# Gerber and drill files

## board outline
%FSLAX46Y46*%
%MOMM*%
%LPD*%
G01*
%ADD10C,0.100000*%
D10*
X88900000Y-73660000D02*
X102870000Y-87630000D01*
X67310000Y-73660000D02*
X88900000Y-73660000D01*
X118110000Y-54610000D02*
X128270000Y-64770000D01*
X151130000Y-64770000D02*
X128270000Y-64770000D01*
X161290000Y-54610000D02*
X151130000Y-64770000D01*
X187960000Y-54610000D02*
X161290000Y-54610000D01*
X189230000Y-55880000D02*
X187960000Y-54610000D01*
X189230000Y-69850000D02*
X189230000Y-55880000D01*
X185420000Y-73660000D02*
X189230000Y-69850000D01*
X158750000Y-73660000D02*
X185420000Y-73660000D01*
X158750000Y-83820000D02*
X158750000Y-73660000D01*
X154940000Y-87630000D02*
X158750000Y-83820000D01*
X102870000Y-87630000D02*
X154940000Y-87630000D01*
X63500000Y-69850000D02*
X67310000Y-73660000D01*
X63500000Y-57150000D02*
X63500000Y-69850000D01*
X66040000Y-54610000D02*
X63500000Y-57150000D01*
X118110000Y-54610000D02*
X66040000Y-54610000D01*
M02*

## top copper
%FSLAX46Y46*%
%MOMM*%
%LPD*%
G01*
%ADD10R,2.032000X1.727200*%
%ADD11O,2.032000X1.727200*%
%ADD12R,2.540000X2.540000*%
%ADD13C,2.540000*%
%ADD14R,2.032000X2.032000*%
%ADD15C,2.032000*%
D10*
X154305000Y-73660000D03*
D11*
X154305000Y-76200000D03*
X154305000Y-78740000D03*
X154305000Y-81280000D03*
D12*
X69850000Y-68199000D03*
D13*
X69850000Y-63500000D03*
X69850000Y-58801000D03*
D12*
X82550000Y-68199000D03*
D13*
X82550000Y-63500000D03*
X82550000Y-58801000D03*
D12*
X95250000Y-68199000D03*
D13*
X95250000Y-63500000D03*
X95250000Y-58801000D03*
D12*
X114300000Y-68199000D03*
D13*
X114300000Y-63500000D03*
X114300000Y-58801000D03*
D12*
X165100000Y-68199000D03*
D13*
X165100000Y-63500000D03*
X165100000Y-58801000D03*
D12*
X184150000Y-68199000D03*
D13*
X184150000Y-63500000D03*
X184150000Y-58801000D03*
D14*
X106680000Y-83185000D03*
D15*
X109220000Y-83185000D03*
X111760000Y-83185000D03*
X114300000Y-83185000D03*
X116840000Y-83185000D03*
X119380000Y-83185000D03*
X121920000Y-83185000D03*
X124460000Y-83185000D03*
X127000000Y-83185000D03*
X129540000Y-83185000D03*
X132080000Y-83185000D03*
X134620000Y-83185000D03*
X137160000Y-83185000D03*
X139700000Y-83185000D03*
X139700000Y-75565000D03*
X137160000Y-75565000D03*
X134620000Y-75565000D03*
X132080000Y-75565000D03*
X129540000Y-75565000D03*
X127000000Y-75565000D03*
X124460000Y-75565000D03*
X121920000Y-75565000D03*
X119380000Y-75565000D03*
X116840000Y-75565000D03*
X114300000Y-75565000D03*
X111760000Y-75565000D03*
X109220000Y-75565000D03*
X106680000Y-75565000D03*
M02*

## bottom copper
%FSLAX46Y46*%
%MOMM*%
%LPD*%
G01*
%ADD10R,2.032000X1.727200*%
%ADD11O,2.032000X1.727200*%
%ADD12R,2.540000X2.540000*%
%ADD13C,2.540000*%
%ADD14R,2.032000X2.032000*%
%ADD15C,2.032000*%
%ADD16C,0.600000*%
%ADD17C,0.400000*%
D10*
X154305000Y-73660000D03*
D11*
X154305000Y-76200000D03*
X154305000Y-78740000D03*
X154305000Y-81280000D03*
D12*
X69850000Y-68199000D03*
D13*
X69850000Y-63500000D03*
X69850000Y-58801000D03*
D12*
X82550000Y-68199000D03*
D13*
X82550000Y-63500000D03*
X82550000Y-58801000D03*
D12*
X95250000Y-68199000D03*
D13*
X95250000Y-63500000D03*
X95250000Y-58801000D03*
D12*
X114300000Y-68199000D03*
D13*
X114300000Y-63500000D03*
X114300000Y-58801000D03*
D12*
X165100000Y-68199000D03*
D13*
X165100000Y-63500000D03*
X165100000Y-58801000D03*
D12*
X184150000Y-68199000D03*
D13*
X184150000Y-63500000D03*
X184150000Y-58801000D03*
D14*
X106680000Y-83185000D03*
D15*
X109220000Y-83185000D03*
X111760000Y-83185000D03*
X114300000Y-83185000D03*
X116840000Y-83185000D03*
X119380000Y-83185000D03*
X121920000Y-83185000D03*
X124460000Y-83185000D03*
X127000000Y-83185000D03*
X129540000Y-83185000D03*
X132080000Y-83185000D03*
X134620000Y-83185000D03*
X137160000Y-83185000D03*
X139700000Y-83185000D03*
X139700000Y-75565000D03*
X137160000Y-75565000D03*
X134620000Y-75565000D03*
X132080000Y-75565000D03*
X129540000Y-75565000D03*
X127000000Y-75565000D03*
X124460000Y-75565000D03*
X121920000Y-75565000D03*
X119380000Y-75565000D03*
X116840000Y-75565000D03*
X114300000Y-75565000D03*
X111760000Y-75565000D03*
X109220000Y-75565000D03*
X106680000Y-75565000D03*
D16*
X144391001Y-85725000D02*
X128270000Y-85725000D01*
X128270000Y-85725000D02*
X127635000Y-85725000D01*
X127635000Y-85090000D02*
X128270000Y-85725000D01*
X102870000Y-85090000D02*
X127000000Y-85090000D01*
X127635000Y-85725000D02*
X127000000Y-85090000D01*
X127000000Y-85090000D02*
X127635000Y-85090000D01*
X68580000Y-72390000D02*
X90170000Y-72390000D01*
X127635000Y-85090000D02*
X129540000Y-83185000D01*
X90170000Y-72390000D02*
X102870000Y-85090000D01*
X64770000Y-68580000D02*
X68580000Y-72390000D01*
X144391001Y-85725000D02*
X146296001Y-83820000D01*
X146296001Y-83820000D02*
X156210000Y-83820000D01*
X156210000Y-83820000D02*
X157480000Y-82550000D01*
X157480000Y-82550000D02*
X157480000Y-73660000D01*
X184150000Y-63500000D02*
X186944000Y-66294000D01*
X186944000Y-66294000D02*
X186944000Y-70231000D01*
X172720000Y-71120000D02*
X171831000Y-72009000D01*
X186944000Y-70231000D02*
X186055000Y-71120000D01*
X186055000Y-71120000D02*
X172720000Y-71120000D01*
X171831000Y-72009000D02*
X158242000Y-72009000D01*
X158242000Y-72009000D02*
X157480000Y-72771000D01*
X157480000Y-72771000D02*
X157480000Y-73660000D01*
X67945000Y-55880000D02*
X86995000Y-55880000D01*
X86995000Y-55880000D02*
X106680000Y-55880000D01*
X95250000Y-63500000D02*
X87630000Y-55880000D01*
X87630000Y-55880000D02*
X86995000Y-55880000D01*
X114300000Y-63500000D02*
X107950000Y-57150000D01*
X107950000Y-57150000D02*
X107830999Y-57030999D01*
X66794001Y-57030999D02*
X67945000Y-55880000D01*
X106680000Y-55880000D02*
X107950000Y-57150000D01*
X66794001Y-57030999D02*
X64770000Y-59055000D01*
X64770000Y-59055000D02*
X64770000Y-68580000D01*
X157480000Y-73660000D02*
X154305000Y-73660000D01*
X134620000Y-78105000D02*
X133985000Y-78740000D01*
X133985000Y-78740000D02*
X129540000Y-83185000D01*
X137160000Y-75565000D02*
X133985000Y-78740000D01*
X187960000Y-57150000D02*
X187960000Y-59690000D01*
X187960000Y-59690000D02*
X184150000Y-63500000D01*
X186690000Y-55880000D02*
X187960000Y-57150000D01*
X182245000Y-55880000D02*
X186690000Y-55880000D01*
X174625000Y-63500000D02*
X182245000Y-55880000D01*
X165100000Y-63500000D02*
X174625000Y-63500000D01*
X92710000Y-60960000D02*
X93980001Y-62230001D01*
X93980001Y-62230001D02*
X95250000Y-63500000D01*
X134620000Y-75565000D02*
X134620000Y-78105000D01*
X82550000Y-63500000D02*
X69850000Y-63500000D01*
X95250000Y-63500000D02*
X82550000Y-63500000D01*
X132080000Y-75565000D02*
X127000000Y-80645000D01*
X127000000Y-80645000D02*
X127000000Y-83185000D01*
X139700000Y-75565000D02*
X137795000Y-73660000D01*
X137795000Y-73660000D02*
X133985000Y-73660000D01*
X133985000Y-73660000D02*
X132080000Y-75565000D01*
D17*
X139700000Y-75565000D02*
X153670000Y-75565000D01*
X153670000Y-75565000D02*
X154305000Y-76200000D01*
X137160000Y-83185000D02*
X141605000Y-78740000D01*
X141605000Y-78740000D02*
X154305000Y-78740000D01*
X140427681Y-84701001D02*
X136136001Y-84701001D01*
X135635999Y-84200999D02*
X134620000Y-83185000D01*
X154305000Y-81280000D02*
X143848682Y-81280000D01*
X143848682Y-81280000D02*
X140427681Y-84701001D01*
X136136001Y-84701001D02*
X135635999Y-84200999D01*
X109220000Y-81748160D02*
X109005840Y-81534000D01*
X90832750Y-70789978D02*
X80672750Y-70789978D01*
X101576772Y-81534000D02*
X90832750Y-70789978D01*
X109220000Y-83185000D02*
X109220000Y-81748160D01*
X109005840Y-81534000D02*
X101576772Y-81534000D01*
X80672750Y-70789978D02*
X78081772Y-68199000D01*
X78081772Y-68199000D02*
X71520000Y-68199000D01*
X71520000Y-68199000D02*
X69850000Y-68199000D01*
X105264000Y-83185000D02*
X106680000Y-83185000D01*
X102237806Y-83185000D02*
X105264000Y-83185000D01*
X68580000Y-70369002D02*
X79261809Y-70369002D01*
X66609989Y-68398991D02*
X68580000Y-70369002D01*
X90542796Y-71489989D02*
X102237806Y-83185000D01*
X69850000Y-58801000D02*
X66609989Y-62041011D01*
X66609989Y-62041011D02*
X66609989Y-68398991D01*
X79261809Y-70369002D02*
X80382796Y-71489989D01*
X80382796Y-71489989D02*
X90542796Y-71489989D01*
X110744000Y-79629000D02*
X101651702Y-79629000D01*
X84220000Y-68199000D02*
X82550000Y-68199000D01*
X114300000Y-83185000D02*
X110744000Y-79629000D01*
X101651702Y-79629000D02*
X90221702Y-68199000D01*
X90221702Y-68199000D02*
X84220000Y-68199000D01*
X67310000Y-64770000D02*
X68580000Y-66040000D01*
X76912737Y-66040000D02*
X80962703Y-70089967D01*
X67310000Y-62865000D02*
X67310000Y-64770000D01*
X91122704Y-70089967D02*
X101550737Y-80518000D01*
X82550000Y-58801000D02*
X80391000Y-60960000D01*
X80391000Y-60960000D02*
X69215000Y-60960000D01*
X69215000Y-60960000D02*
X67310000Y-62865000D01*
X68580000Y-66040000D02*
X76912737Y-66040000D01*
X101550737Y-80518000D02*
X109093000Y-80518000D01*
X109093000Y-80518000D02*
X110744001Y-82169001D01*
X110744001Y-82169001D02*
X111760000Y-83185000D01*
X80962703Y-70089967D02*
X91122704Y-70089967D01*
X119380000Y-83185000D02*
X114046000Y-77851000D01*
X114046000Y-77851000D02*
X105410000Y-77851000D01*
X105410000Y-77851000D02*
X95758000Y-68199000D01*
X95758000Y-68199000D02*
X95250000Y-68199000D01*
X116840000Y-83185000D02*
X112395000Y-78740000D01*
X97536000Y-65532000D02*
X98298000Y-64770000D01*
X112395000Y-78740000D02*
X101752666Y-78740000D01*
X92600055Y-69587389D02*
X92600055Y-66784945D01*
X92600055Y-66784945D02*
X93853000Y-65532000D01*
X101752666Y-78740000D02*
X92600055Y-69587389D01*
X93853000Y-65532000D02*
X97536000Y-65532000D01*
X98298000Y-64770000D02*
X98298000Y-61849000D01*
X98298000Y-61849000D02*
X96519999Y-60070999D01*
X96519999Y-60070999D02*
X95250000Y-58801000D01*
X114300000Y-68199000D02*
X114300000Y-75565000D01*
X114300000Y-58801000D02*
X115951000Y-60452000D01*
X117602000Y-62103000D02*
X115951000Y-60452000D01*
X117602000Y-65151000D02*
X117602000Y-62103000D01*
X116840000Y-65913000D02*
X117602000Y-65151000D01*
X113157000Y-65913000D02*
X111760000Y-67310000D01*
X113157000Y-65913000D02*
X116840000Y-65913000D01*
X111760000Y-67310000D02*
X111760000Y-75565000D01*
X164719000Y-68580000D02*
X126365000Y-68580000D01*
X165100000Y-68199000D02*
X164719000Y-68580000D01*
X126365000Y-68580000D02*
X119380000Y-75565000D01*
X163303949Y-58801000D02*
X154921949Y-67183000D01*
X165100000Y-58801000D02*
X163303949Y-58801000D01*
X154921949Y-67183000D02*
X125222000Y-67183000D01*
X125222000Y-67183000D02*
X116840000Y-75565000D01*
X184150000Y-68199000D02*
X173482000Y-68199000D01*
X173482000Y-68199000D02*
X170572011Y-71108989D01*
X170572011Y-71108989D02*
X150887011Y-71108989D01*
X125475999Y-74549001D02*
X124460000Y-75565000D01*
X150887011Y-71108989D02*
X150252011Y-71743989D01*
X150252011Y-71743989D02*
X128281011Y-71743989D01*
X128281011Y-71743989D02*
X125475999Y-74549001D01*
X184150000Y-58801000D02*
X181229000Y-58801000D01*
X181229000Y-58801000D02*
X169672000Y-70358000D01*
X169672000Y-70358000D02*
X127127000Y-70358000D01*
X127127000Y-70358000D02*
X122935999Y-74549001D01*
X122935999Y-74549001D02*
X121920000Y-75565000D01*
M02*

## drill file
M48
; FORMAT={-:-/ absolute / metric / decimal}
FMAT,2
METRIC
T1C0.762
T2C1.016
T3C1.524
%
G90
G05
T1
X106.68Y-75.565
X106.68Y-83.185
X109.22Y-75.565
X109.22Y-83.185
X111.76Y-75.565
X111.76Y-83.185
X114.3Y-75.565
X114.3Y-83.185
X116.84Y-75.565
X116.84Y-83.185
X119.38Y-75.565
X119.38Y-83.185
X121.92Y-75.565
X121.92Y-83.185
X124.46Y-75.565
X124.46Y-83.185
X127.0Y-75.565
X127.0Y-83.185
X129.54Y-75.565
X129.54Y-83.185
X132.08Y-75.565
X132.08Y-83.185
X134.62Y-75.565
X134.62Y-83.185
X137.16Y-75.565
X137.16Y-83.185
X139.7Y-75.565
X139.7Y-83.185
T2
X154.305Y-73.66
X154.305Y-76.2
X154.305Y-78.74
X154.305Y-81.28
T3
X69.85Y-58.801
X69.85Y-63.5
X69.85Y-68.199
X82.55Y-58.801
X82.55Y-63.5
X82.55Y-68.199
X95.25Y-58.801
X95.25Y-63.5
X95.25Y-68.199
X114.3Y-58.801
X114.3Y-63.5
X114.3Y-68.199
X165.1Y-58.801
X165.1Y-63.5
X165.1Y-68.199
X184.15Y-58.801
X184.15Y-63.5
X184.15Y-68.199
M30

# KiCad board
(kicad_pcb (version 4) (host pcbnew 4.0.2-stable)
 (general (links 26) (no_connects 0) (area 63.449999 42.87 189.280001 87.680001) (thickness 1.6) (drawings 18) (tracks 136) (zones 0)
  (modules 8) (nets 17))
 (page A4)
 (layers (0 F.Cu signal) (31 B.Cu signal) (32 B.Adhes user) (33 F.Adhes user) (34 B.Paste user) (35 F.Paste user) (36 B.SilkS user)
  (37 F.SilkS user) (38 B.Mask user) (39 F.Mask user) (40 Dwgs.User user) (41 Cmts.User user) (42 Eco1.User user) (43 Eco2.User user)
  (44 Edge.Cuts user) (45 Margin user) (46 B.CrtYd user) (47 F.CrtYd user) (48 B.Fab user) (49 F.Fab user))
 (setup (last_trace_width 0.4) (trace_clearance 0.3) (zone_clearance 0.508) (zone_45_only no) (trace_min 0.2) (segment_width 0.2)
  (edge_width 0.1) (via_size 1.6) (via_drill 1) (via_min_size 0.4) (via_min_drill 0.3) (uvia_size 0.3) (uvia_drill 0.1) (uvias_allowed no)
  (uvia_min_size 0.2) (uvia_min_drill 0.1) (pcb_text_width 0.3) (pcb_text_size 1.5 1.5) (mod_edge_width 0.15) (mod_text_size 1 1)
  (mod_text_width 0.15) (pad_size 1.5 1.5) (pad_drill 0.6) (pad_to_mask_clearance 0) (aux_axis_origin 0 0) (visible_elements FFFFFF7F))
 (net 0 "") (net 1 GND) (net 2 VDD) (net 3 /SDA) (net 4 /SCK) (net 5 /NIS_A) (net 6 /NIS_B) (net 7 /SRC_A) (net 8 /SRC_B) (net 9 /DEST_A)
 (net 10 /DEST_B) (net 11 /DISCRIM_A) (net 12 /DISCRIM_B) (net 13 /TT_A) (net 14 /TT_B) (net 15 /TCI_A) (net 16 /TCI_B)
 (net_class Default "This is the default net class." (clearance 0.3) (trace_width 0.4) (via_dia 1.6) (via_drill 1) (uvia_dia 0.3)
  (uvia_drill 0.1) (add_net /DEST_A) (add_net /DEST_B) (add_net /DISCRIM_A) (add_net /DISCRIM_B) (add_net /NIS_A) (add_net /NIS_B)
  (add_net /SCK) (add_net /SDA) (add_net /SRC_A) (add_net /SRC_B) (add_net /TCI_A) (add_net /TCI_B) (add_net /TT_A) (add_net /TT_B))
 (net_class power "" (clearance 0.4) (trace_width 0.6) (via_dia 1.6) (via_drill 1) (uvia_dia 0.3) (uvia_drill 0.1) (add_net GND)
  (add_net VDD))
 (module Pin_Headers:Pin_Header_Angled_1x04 (layer F.Cu) (at 154.305 73.66)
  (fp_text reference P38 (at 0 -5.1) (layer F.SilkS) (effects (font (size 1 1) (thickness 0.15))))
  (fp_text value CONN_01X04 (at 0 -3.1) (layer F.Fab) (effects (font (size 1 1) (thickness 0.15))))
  (pad 1 thru_hole rect (at 0 0) (size 2.032 1.7272) (drill 1.016) (layers *.Cu *.Mask F.SilkS) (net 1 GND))
  (pad 2 thru_hole oval (at 0 2.54) (size 2.032 1.7272) (drill 1.016) (layers *.Cu *.Mask F.SilkS) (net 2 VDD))
  (pad 3 thru_hole oval (at 0 5.08) (size 2.032 1.7272) (drill 1.016) (layers *.Cu *.Mask F.SilkS) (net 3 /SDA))
  (pad 4 thru_hole oval (at 0 7.62) (size 2.032 1.7272) (drill 1.016) (layers *.Cu *.Mask F.SilkS) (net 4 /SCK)))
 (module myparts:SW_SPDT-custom (layer F.Cu) (at 69.85 63.5 90)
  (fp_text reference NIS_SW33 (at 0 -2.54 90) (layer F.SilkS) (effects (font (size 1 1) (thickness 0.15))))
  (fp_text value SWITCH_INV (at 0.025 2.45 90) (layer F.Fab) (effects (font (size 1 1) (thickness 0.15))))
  (pad 1 thru_hole rect (at -4.699 0 90) (size 2.54 2.54) (drill 1.524) (layers *.Cu *.Mask F.SilkS) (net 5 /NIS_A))
  (pad 2 thru_hole circle (at 0 0 90) (size 2.54 2.54) (drill 1.524) (layers *.Cu *.Mask F.SilkS) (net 1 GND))
  (pad 3 thru_hole circle (at 4.699 0 90) (size 2.54 2.54) (drill 1.524) (layers *.Cu *.Mask F.SilkS) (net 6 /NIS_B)))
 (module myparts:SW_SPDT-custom (layer F.Cu) (at 82.55 63.5 90)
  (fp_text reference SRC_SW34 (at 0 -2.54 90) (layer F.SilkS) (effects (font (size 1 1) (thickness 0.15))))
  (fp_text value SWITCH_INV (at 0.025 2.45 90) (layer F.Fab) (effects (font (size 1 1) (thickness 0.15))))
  (pad 1 thru_hole rect (at -4.699 0 90) (size 2.54 2.54) (drill 1.524) (layers *.Cu *.Mask F.SilkS) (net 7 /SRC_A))
  (pad 2 thru_hole circle (at 0 0 90) (size 2.54 2.54) (drill 1.524) (layers *.Cu *.Mask F.SilkS) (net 1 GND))
  (pad 3 thru_hole circle (at 4.699 0 90) (size 2.54 2.54) (drill 1.524) (layers *.Cu *.Mask F.SilkS) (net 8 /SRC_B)))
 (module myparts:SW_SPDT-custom (layer F.Cu) (at 95.25 63.5 90)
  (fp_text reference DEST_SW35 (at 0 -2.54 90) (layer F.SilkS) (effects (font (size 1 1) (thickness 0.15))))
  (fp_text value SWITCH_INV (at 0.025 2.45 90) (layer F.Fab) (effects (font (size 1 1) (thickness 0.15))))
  (pad 1 thru_hole rect (at -4.699 0 90) (size 2.54 2.54) (drill 1.524) (layers *.Cu *.Mask F.SilkS) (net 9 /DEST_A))
  (pad 2 thru_hole circle (at 0 0 90) (size 2.54 2.54) (drill 1.524) (layers *.Cu *.Mask F.SilkS) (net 1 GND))
  (pad 3 thru_hole circle (at 4.699 0 90) (size 2.54 2.54) (drill 1.524) (layers *.Cu *.Mask F.SilkS) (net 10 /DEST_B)))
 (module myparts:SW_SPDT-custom (layer F.Cu) (at 114.3 63.5 90)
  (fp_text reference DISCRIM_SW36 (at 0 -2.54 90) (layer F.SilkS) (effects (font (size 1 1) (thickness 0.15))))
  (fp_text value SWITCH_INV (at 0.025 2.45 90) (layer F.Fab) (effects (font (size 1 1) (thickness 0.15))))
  (pad 1 thru_hole rect (at -4.699 0 90) (size 2.54 2.54) (drill 1.524) (layers *.Cu *.Mask F.SilkS) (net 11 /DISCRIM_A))
  (pad 2 thru_hole circle (at 0 0 90) (size 2.54 2.54) (drill 1.524) (layers *.Cu *.Mask F.SilkS) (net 1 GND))
  (pad 3 thru_hole circle (at 4.699 0 90) (size 2.54 2.54) (drill 1.524) (layers *.Cu *.Mask F.SilkS) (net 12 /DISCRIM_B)))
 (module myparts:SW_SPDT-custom (layer F.Cu) (at 165.1 63.5 90)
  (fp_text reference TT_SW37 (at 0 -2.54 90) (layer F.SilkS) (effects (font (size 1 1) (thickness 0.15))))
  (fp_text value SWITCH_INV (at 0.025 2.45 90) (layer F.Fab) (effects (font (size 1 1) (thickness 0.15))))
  (pad 1 thru_hole rect (at -4.699 0 90) (size 2.54 2.54) (drill 1.524) (layers *.Cu *.Mask F.SilkS) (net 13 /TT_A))
  (pad 2 thru_hole circle (at 0 0 90) (size 2.54 2.54) (drill 1.524) (layers *.Cu *.Mask F.SilkS) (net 1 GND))
  (pad 3 thru_hole circle (at 4.699 0 90) (size 2.54 2.54) (drill 1.524) (layers *.Cu *.Mask F.SilkS) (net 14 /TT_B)))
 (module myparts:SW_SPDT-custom (layer F.Cu) (at 184.15 63.5 90)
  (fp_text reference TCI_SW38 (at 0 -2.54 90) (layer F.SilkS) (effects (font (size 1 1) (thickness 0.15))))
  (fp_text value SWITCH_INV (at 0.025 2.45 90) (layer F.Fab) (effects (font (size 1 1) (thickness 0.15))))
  (pad 1 thru_hole rect (at -4.699 0 90) (size 2.54 2.54) (drill 1.524) (layers *.Cu *.Mask F.SilkS) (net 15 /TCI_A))
  (pad 2 thru_hole circle (at 0 0 90) (size 2.54 2.54) (drill 1.524) (layers *.Cu *.Mask F.SilkS) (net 1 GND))
  (pad 3 thru_hole circle (at 4.699 0 90) (size 2.54 2.54) (drill 1.524) (layers *.Cu *.Mask F.SilkS) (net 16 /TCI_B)))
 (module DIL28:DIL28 (layer F.Cu) (at 106.68 83.185)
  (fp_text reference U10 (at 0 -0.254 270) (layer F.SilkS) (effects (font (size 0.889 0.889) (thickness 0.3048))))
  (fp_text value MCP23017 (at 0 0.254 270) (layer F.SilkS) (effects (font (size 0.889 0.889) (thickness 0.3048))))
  (pad 1 thru_hole rect (at 0 0) (size 2.032 2.032) (drill 0.762) (layers *.Cu *.Mask F.SilkS) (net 6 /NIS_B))
  (pad 2 thru_hole circle (at 2.54 0) (size 2.032 2.032) (drill 0.762) (layers *.Cu *.Mask F.SilkS) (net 5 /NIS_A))
  (pad 3 thru_hole circle (at 5.08 0) (size 2.032 2.032) (drill 0.762) (layers *.Cu *.Mask F.SilkS) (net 8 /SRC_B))
  (pad 4 thru_hole circle (at 7.62 0) (size 2.032 2.032) (drill 0.762) (layers *.Cu *.Mask F.SilkS) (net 7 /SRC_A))
  (pad 5 thru_hole circle (at 10.16 0) (size 2.032 2.032) (drill 0.762) (layers *.Cu *.Mask F.SilkS) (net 10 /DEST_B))
  (pad 6 thru_hole circle (at 12.7 0) (size 2.032 2.032) (drill 0.762) (layers *.Cu *.Mask F.SilkS) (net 9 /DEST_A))
  (pad 7 thru_hole circle (at 15.24 0) (size 2.032 2.032) (drill 0.762) (layers *.Cu *.Mask F.SilkS))
  (pad 8 thru_hole circle (at 17.78 0) (size 2.032 2.032) (drill 0.762) (layers *.Cu *.Mask F.SilkS))
  (pad 9 thru_hole circle (at 20.32 0) (size 2.032 2.032) (drill 0.762) (layers *.Cu *.Mask F.SilkS) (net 2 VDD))
  (pad 10 thru_hole circle (at 22.86 0) (size 2.032 2.032) (drill 0.762) (layers *.Cu *.Mask F.SilkS) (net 1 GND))
  (pad 11 thru_hole circle (at 25.4 0) (size 2.032 2.032) (drill 0.762) (layers *.Cu *.Mask F.SilkS))
  (pad 12 thru_hole circle (at 27.94 0) (size 2.032 2.032) (drill 0.762) (layers *.Cu *.Mask F.SilkS) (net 4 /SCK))
  (pad 13 thru_hole circle (at 30.48 0) (size 2.032 2.032) (drill 0.762) (layers *.Cu *.Mask F.SilkS) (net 3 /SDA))
  (pad 14 thru_hole circle (at 33.02 0) (size 2.032 2.032) (drill 0.762) (layers *.Cu *.Mask F.SilkS))
  (pad 15 thru_hole circle (at 33.02 -7.62 180) (size 2.032 2.032) (drill 0.762) (layers *.Cu *.Mask F.SilkS) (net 2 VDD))
  (pad 16 thru_hole circle (at 30.48 -7.62 180) (size 2.032 2.032) (drill 0.762) (layers *.Cu *.Mask F.SilkS) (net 1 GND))
  (pad 17 thru_hole circle (at 27.94 -7.62 180) (size 2.032 2.032) (drill 0.762) (layers *.Cu *.Mask F.SilkS) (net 1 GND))
  (pad 18 thru_hole circle (at 25.4 -7.62 180) (size 2.032 2.032) (drill 0.762) (layers *.Cu *.Mask F.SilkS) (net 2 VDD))
  (pad 19 thru_hole circle (at 22.86 -7.62 180) (size 2.032 2.032) (drill 0.762) (layers *.Cu *.Mask F.SilkS))
  (pad 20 thru_hole circle (at 20.32 -7.62 180) (size 2.032 2.032) (drill 0.762) (layers *.Cu *.Mask F.SilkS))
  (pad 21 thru_hole circle (at 17.78 -7.62 180) (size 2.032 2.032) (drill 0.762) (layers *.Cu *.Mask F.SilkS) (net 15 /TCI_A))
  (pad 22 thru_hole circle (at 15.24 -7.62 180) (size 2.032 2.032) (drill 0.762) (layers *.Cu *.Mask F.SilkS) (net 16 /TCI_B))
  (pad 23 thru_hole circle (at 12.7 -7.62 180) (size 2.032 2.032) (drill 0.762) (layers *.Cu *.Mask F.SilkS) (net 13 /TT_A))
  (pad 24 thru_hole circle (at 10.16 -7.62 180) (size 2.032 2.032) (drill 0.762) (layers *.Cu *.Mask F.SilkS) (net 14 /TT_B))
  (pad 25 thru_hole circle (at 7.62 -7.62 180) (size 2.032 2.032) (drill 0.762) (layers *.Cu *.Mask F.SilkS) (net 11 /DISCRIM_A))
  (pad 26 thru_hole circle (at 5.08 -7.62 180) (size 2.032 2.032) (drill 0.762) (layers *.Cu *.Mask F.SilkS) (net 12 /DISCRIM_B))
  (pad 27 thru_hole circle (at 2.54 -7.62 180) (size 2.032 2.032) (drill 0.762) (layers *.Cu *.Mask F.SilkS))
  (pad 28 thru_hole circle (at 0 -7.62 180) (size 2.032 2.032) (drill 0.762) (layers *.Cu *.Mask F.SilkS)))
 (gr_line (start 88.9 73.66) (end 102.87 87.63) (layer Edge.Cuts) (width 0.1))
 (gr_line (start 67.31 73.66) (end 88.9 73.66) (layer Edge.Cuts) (width 0.1))
 (gr_line (start 118.11 54.61) (end 128.27 64.77) (layer Edge.Cuts) (width 0.1))
 (gr_line (start 151.13 64.77) (end 128.27 64.77) (layer Edge.Cuts) (width 0.1))
 (gr_line (start 161.29 54.61) (end 151.13 64.77) (layer Edge.Cuts) (width 0.1))
 (gr_line (start 187.96 54.61) (end 161.29 54.61) (layer Edge.Cuts) (width 0.1))
 (gr_line (start 189.23 55.88) (end 187.96 54.61) (layer Edge.Cuts) (width 0.1))
 (gr_line (start 189.23 69.85) (end 189.23 55.88) (layer Edge.Cuts) (width 0.1))
 (gr_line (start 185.42 73.66) (end 189.23 69.85) (layer Edge.Cuts) (width 0.1))
 (gr_line (start 158.75 73.66) (end 185.42 73.66) (layer Edge.Cuts) (width 0.1))
 (gr_line (start 158.75 83.82) (end 158.75 73.66) (layer Edge.Cuts) (width 0.1))
 (gr_line (start 154.94 87.63) (end 158.75 83.82) (layer Edge.Cuts) (width 0.1))
 (gr_line (start 102.87 87.63) (end 154.94 87.63) (layer Edge.Cuts) (width 0.1))
 (gr_line (start 63.5 69.85) (end 67.31 73.66) (layer Edge.Cuts) (width 0.1))
 (gr_line (start 63.5 57.15) (end 63.5 69.85) (layer Edge.Cuts) (width 0.1))
 (gr_line (start 66.04 54.61) (end 63.5 57.15) (layer Edge.Cuts) (width 0.1))
 (gr_line (start 118.11 54.61) (end 66.04 54.61) (layer Edge.Cuts) (width 0.1))
 (segment (start 144.391001 85.725) (end 128.27 85.725) (width 0.6) (layer B.Cu) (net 1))
 (segment (start 128.27 85.725) (end 127.635 85.725) (width 0.6) (layer B.Cu) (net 1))
 (segment (start 127.635 85.09) (end 128.27 85.725) (width 0.6) (layer B.Cu) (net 1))
 (segment (start 102.87 85.09) (end 127 85.09) (width 0.6) (layer B.Cu) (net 1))
 (segment (start 127.635 85.725) (end 127 85.09) (width 0.6) (layer B.Cu) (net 1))
 (segment (start 127 85.09) (end 127.635 85.09) (width 0.6) (layer B.Cu) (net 1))
 (segment (start 68.58 72.39) (end 90.17 72.39) (width 0.6) (layer B.Cu) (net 1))
 (segment (start 127.635 85.09) (end 129.54 83.185) (width 0.6) (layer B.Cu) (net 1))
 (segment (start 90.17 72.39) (end 102.87 85.09) (width 0.6) (layer B.Cu) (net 1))
 (segment (start 64.77 68.58) (end 68.58 72.39) (width 0.6) (layer B.Cu) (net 1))
 (segment (start 144.391001 85.725) (end 146.296001 83.82) (width 0.6) (layer B.Cu) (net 1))
 (segment (start 146.296001 83.82) (end 156.21 83.82) (width 0.6) (layer B.Cu) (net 1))
 (segment (start 156.21 83.82) (end 157.48 82.55) (width 0.6) (layer B.Cu) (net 1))
 (segment (start 157.48 82.55) (end 157.48 73.66) (width 0.6) (layer B.Cu) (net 1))
 (segment (start 184.15 63.5) (end 186.944 66.294) (width 0.6) (layer B.Cu) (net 1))
 (segment (start 186.944 66.294) (end 186.944 70.231) (width 0.6) (layer B.Cu) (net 1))
 (segment (start 172.72 71.12) (end 171.831 72.009) (width 0.6) (layer B.Cu) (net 1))
 (segment (start 186.944 70.231) (end 186.055 71.12) (width 0.6) (layer B.Cu) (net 1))
 (segment (start 186.055 71.12) (end 172.72 71.12) (width 0.6) (layer B.Cu) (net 1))
 (segment (start 171.831 72.009) (end 158.242 72.009) (width 0.6) (layer B.Cu) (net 1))
 (segment (start 158.242 72.009) (end 157.48 72.771) (width 0.6) (layer B.Cu) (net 1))
 (segment (start 157.48 72.771) (end 157.48 73.66) (width 0.6) (layer B.Cu) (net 1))
 (segment (start 67.945 55.88) (end 86.995 55.88) (width 0.6) (layer B.Cu) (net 1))
 (segment (start 86.995 55.88) (end 106.68 55.88) (width 0.6) (layer B.Cu) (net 1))
 (segment (start 95.25 63.5) (end 87.63 55.88) (width 0.6) (layer B.Cu) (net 1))
 (segment (start 87.63 55.88) (end 86.995 55.88) (width 0.6) (layer B.Cu) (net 1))
 (segment (start 114.3 63.5) (end 107.95 57.15) (width 0.6) (layer B.Cu) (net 1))
 (segment (start 107.95 57.15) (end 107.830999 57.030999) (width 0.6) (layer B.Cu) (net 1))
 (segment (start 66.794001 57.030999) (end 67.945 55.88) (width 0.6) (layer B.Cu) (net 1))
 (segment (start 106.68 55.88) (end 107.95 57.15) (width 0.6) (layer B.Cu) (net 1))
 (segment (start 66.794001 57.030999) (end 64.77 59.055) (width 0.6) (layer B.Cu) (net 1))
 (segment (start 64.77 59.055) (end 64.77 68.58) (width 0.6) (layer B.Cu) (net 1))
 (segment (start 157.48 73.66) (end 154.305 73.66) (width 0.6) (layer B.Cu) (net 1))
 (segment (start 134.62 78.105) (end 133.985 78.74) (width 0.6) (layer B.Cu) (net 1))
 (segment (start 133.985 78.74) (end 129.54 83.185) (width 0.6) (layer B.Cu) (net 1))
 (segment (start 137.16 75.565) (end 133.985 78.74) (width 0.6) (layer B.Cu) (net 1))
 (segment (start 187.96 57.15) (end 187.96 59.69) (width 0.6) (layer B.Cu) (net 1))
 (segment (start 187.96 59.69) (end 184.15 63.5) (width 0.6) (layer B.Cu) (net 1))
 (segment (start 186.69 55.88) (end 187.96 57.15) (width 0.6) (layer B.Cu) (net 1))
 (segment (start 182.245 55.88) (end 186.69 55.88) (width 0.6) (layer B.Cu) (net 1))
 (segment (start 174.625 63.5) (end 182.245 55.88) (width 0.6) (layer B.Cu) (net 1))
 (segment (start 165.1 63.5) (end 174.625 63.5) (width 0.6) (layer B.Cu) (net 1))
 (segment (start 92.71 60.96) (end 93.980001 62.230001) (width 0.6) (layer B.Cu) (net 1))
 (segment (start 93.980001 62.230001) (end 95.25 63.5) (width 0.6) (layer B.Cu) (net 1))
 (segment (start 134.62 75.565) (end 134.62 78.105) (width 0.6) (layer B.Cu) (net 1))
 (segment (start 82.55 63.5) (end 69.85 63.5) (width 0.6) (layer B.Cu) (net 1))
 (segment (start 95.25 63.5) (end 82.55 63.5) (width 0.6) (layer B.Cu) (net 1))
 (segment (start 132.08 75.565) (end 127 80.645) (width 0.6) (layer B.Cu) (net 2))
 (segment (start 127 80.645) (end 127 83.185) (width 0.6) (layer B.Cu) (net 2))
 (segment (start 139.7 75.565) (end 137.795 73.66) (width 0.6) (layer B.Cu) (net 2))
 (segment (start 137.795 73.66) (end 133.985 73.66) (width 0.6) (layer B.Cu) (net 2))
 (segment (start 133.985 73.66) (end 132.08 75.565) (width 0.6) (layer B.Cu) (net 2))
 (segment (start 139.7 75.565) (end 153.67 75.565) (width 0.4) (layer B.Cu) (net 2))
 (segment (start 153.67 75.565) (end 154.305 76.2) (width 0.4) (layer B.Cu) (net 2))
 (segment (start 137.16 83.185) (end 141.605 78.74) (width 0.4) (layer B.Cu) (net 3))
 (segment (start 141.605 78.74) (end 154.305 78.74) (width 0.4) (layer B.Cu) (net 3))
 (segment (start 140.427681 84.701001) (end 136.136001 84.701001) (width 0.4) (layer B.Cu) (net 4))
 (segment (start 135.635999 84.200999) (end 134.62 83.185) (width 0.4) (layer B.Cu) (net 4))
 (segment (start 154.305 81.28) (end 143.848682 81.28) (width 0.4) (layer B.Cu) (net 4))
 (segment (start 143.848682 81.28) (end 140.427681 84.701001) (width 0.4) (layer B.Cu) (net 4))
 (segment (start 136.136001 84.701001) (end 135.635999 84.200999) (width 0.4) (layer B.Cu) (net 4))
 (segment (start 109.22 81.74816) (end 109.00584 81.534) (width 0.4) (layer B.Cu) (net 5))
 (segment (start 90.83275 70.789978) (end 80.67275 70.789978) (width 0.4) (layer B.Cu) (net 5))
 (segment (start 101.576772 81.534) (end 90.83275 70.789978) (width 0.4) (layer B.Cu) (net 5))
 (segment (start 109.22 83.185) (end 109.22 81.74816) (width 0.4) (layer B.Cu) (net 5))
 (segment (start 109.00584 81.534) (end 101.576772 81.534) (width 0.4) (layer B.Cu) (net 5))
 (segment (start 80.67275 70.789978) (end 78.081772 68.199) (width 0.4) (layer B.Cu) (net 5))
 (segment (start 78.081772 68.199) (end 71.52 68.199) (width 0.4) (layer B.Cu) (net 5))
 (segment (start 71.52 68.199) (end 69.85 68.199) (width 0.4) (layer B.Cu) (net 5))
 (segment (start 105.264 83.185) (end 106.68 83.185) (width 0.4) (layer B.Cu) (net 6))
 (segment (start 102.237806 83.185) (end 105.264 83.185) (width 0.4) (layer B.Cu) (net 6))
 (segment (start 68.58 70.369002) (end 79.261809 70.369002) (width 0.4) (layer B.Cu) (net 6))
 (segment (start 66.609989 68.398991) (end 68.58 70.369002) (width 0.4) (layer B.Cu) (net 6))
 (segment (start 90.542796 71.489989) (end 102.237806 83.185) (width 0.4) (layer B.Cu) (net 6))
 (segment (start 69.85 58.801) (end 66.609989 62.041011) (width 0.4) (layer B.Cu) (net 6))
 (segment (start 66.609989 62.041011) (end 66.609989 68.398991) (width 0.4) (layer B.Cu) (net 6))
 (segment (start 79.261809 70.369002) (end 80.382796 71.489989) (width 0.4) (layer B.Cu) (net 6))
 (segment (start 80.382796 71.489989) (end 90.542796 71.489989) (width 0.4) (layer B.Cu) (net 6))
 (segment (start 110.744 79.629) (end 101.651702 79.629) (width 0.4) (layer B.Cu) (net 7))
 (segment (start 84.22 68.199) (end 82.55 68.199) (width 0.4) (layer B.Cu) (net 7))
 (segment (start 114.3 83.185) (end 110.744 79.629) (width 0.4) (layer B.Cu) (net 7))
 (segment (start 101.651702 79.629) (end 90.221702 68.199) (width 0.4) (layer B.Cu) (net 7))
 (segment (start 90.221702 68.199) (end 84.22 68.199) (width 0.4) (layer B.Cu) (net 7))
 (segment (start 67.31 64.77) (end 68.58 66.04) (width 0.4) (layer B.Cu) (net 8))
 (segment (start 76.912737 66.04) (end 80.962703 70.089967) (width 0.4) (layer B.Cu) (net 8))
 (segment (start 67.31 62.865) (end 67.31 64.77) (width 0.4) (layer B.Cu) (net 8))
 (segment (start 91.122704 70.089967) (end 101.550737 80.518) (width 0.4) (layer B.Cu) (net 8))
 (segment (start 82.55 58.801) (end 80.391 60.96) (width 0.4) (layer B.Cu) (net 8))
 (segment (start 80.391 60.96) (end 69.215 60.96) (width 0.4) (layer B.Cu) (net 8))
 (segment (start 69.215 60.96) (end 67.31 62.865) (width 0.4) (layer B.Cu) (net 8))
 (segment (start 68.58 66.04) (end 76.912737 66.04) (width 0.4) (layer B.Cu) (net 8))
 (segment (start 101.550737 80.518) (end 109.093 80.518) (width 0.4) (layer B.Cu) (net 8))
 (segment (start 109.093 80.518) (end 110.744001 82.169001) (width 0.4) (layer B.Cu) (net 8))
 (segment (start 110.744001 82.169001) (end 111.76 83.185) (width 0.4) (layer B.Cu) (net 8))
 (segment (start 80.962703 70.089967) (end 91.122704 70.089967) (width 0.4) (layer B.Cu) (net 8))
 (segment (start 119.38 83.185) (end 114.046 77.851) (width 0.4) (layer B.Cu) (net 9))
 (segment (start 114.046 77.851) (end 105.41 77.851) (width 0.4) (layer B.Cu) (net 9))
 (segment (start 105.41 77.851) (end 95.758 68.199) (width 0.4) (layer B.Cu) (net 9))
 (segment (start 95.758 68.199) (end 95.25 68.199) (width 0.4) (layer B.Cu) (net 9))
 (segment (start 116.84 83.185) (end 112.395 78.74) (width 0.4) (layer B.Cu) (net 10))
 (segment (start 97.536 65.532) (end 98.298 64.77) (width 0.4) (layer B.Cu) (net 10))
 (segment (start 112.395 78.74) (end 101.752666 78.74) (width 0.4) (layer B.Cu) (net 10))
 (segment (start 92.600055 69.587389) (end 92.600055 66.784945) (width 0.4) (layer B.Cu) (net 10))
 (segment (start 92.600055 66.784945) (end 93.853 65.532) (width 0.4) (layer B.Cu) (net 10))
 (segment (start 101.752666 78.74) (end 92.600055 69.587389) (width 0.4) (layer B.Cu) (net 10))
 (segment (start 93.853 65.532) (end 97.536 65.532) (width 0.4) (layer B.Cu) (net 10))
 (segment (start 98.298 64.77) (end 98.298 61.849) (width 0.4) (layer B.Cu) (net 10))
 (segment (start 98.298 61.849) (end 96.519999 60.070999) (width 0.4) (layer B.Cu) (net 10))
 (segment (start 96.519999 60.070999) (end 95.25 58.801) (width 0.4) (layer B.Cu) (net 10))
 (segment (start 114.3 68.199) (end 114.3 75.565) (width 0.4) (layer B.Cu) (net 11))
 (segment (start 114.3 58.801) (end 115.951 60.452) (width 0.4) (layer B.Cu) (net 12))
 (segment (start 117.602 62.103) (end 115.951 60.452) (width 0.4) (layer B.Cu) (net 12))
 (segment (start 117.602 65.151) (end 117.602 62.103) (width 0.4) (layer B.Cu) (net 12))
 (segment (start 116.84 65.913) (end 117.602 65.151) (width 0.4) (layer B.Cu) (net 12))
 (segment (start 113.157 65.913) (end 111.76 67.31) (width 0.4) (layer B.Cu) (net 12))
 (segment (start 113.157 65.913) (end 116.84 65.913) (width 0.4) (layer B.Cu) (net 12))
 (segment (start 111.76 67.31) (end 111.76 75.565) (width 0.4) (layer B.Cu) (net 12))
 (segment (start 164.719 68.58) (end 126.365 68.58) (width 0.4) (layer B.Cu) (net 13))
 (segment (start 165.1 68.199) (end 164.719 68.58) (width 0.4) (layer B.Cu) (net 13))
 (segment (start 126.365 68.58) (end 119.38 75.565) (width 0.4) (layer B.Cu) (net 13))
 (segment (start 163.303949 58.801) (end 154.921949 67.183) (width 0.4) (layer B.Cu) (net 14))
 (segment (start 165.1 58.801) (end 163.303949 58.801) (width 0.4) (layer B.Cu) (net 14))
 (segment (start 154.921949 67.183) (end 125.222 67.183) (width 0.4) (layer B.Cu) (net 14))
 (segment (start 125.222 67.183) (end 116.84 75.565) (width 0.4) (layer B.Cu) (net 14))
 (segment (start 184.15 68.199) (end 173.482 68.199) (width 0.4) (layer B.Cu) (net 15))
 (segment (start 173.482 68.199) (end 170.572011 71.108989) (width 0.4) (layer B.Cu) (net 15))
 (segment (start 170.572011 71.108989) (end 150.887011 71.108989) (width 0.4) (layer B.Cu) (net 15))
 (segment (start 125.475999 74.549001) (end 124.46 75.565) (width 0.4) (layer B.Cu) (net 15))
 (segment (start 150.887011 71.108989) (end 150.252011 71.743989) (width 0.4) (layer B.Cu) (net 15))
 (segment (start 150.252011 71.743989) (end 128.281011 71.743989) (width 0.4) (layer B.Cu) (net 15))
 (segment (start 128.281011 71.743989) (end 125.475999 74.549001) (width 0.4) (layer B.Cu) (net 15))
 (segment (start 184.15 58.801) (end 181.229 58.801) (width 0.4) (layer B.Cu) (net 16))
 (segment (start 181.229 58.801) (end 169.672 70.358) (width 0.4) (layer B.Cu) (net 16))
 (segment (start 169.672 70.358) (end 127.127 70.358) (width 0.4) (layer B.Cu) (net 16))
 (segment (start 127.127 70.358) (end 122.935999 74.549001) (width 0.4) (layer B.Cu) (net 16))
 (segment (start 122.935999 74.549001) (end 121.92 75.565) (width 0.4) (layer B.Cu) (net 16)))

